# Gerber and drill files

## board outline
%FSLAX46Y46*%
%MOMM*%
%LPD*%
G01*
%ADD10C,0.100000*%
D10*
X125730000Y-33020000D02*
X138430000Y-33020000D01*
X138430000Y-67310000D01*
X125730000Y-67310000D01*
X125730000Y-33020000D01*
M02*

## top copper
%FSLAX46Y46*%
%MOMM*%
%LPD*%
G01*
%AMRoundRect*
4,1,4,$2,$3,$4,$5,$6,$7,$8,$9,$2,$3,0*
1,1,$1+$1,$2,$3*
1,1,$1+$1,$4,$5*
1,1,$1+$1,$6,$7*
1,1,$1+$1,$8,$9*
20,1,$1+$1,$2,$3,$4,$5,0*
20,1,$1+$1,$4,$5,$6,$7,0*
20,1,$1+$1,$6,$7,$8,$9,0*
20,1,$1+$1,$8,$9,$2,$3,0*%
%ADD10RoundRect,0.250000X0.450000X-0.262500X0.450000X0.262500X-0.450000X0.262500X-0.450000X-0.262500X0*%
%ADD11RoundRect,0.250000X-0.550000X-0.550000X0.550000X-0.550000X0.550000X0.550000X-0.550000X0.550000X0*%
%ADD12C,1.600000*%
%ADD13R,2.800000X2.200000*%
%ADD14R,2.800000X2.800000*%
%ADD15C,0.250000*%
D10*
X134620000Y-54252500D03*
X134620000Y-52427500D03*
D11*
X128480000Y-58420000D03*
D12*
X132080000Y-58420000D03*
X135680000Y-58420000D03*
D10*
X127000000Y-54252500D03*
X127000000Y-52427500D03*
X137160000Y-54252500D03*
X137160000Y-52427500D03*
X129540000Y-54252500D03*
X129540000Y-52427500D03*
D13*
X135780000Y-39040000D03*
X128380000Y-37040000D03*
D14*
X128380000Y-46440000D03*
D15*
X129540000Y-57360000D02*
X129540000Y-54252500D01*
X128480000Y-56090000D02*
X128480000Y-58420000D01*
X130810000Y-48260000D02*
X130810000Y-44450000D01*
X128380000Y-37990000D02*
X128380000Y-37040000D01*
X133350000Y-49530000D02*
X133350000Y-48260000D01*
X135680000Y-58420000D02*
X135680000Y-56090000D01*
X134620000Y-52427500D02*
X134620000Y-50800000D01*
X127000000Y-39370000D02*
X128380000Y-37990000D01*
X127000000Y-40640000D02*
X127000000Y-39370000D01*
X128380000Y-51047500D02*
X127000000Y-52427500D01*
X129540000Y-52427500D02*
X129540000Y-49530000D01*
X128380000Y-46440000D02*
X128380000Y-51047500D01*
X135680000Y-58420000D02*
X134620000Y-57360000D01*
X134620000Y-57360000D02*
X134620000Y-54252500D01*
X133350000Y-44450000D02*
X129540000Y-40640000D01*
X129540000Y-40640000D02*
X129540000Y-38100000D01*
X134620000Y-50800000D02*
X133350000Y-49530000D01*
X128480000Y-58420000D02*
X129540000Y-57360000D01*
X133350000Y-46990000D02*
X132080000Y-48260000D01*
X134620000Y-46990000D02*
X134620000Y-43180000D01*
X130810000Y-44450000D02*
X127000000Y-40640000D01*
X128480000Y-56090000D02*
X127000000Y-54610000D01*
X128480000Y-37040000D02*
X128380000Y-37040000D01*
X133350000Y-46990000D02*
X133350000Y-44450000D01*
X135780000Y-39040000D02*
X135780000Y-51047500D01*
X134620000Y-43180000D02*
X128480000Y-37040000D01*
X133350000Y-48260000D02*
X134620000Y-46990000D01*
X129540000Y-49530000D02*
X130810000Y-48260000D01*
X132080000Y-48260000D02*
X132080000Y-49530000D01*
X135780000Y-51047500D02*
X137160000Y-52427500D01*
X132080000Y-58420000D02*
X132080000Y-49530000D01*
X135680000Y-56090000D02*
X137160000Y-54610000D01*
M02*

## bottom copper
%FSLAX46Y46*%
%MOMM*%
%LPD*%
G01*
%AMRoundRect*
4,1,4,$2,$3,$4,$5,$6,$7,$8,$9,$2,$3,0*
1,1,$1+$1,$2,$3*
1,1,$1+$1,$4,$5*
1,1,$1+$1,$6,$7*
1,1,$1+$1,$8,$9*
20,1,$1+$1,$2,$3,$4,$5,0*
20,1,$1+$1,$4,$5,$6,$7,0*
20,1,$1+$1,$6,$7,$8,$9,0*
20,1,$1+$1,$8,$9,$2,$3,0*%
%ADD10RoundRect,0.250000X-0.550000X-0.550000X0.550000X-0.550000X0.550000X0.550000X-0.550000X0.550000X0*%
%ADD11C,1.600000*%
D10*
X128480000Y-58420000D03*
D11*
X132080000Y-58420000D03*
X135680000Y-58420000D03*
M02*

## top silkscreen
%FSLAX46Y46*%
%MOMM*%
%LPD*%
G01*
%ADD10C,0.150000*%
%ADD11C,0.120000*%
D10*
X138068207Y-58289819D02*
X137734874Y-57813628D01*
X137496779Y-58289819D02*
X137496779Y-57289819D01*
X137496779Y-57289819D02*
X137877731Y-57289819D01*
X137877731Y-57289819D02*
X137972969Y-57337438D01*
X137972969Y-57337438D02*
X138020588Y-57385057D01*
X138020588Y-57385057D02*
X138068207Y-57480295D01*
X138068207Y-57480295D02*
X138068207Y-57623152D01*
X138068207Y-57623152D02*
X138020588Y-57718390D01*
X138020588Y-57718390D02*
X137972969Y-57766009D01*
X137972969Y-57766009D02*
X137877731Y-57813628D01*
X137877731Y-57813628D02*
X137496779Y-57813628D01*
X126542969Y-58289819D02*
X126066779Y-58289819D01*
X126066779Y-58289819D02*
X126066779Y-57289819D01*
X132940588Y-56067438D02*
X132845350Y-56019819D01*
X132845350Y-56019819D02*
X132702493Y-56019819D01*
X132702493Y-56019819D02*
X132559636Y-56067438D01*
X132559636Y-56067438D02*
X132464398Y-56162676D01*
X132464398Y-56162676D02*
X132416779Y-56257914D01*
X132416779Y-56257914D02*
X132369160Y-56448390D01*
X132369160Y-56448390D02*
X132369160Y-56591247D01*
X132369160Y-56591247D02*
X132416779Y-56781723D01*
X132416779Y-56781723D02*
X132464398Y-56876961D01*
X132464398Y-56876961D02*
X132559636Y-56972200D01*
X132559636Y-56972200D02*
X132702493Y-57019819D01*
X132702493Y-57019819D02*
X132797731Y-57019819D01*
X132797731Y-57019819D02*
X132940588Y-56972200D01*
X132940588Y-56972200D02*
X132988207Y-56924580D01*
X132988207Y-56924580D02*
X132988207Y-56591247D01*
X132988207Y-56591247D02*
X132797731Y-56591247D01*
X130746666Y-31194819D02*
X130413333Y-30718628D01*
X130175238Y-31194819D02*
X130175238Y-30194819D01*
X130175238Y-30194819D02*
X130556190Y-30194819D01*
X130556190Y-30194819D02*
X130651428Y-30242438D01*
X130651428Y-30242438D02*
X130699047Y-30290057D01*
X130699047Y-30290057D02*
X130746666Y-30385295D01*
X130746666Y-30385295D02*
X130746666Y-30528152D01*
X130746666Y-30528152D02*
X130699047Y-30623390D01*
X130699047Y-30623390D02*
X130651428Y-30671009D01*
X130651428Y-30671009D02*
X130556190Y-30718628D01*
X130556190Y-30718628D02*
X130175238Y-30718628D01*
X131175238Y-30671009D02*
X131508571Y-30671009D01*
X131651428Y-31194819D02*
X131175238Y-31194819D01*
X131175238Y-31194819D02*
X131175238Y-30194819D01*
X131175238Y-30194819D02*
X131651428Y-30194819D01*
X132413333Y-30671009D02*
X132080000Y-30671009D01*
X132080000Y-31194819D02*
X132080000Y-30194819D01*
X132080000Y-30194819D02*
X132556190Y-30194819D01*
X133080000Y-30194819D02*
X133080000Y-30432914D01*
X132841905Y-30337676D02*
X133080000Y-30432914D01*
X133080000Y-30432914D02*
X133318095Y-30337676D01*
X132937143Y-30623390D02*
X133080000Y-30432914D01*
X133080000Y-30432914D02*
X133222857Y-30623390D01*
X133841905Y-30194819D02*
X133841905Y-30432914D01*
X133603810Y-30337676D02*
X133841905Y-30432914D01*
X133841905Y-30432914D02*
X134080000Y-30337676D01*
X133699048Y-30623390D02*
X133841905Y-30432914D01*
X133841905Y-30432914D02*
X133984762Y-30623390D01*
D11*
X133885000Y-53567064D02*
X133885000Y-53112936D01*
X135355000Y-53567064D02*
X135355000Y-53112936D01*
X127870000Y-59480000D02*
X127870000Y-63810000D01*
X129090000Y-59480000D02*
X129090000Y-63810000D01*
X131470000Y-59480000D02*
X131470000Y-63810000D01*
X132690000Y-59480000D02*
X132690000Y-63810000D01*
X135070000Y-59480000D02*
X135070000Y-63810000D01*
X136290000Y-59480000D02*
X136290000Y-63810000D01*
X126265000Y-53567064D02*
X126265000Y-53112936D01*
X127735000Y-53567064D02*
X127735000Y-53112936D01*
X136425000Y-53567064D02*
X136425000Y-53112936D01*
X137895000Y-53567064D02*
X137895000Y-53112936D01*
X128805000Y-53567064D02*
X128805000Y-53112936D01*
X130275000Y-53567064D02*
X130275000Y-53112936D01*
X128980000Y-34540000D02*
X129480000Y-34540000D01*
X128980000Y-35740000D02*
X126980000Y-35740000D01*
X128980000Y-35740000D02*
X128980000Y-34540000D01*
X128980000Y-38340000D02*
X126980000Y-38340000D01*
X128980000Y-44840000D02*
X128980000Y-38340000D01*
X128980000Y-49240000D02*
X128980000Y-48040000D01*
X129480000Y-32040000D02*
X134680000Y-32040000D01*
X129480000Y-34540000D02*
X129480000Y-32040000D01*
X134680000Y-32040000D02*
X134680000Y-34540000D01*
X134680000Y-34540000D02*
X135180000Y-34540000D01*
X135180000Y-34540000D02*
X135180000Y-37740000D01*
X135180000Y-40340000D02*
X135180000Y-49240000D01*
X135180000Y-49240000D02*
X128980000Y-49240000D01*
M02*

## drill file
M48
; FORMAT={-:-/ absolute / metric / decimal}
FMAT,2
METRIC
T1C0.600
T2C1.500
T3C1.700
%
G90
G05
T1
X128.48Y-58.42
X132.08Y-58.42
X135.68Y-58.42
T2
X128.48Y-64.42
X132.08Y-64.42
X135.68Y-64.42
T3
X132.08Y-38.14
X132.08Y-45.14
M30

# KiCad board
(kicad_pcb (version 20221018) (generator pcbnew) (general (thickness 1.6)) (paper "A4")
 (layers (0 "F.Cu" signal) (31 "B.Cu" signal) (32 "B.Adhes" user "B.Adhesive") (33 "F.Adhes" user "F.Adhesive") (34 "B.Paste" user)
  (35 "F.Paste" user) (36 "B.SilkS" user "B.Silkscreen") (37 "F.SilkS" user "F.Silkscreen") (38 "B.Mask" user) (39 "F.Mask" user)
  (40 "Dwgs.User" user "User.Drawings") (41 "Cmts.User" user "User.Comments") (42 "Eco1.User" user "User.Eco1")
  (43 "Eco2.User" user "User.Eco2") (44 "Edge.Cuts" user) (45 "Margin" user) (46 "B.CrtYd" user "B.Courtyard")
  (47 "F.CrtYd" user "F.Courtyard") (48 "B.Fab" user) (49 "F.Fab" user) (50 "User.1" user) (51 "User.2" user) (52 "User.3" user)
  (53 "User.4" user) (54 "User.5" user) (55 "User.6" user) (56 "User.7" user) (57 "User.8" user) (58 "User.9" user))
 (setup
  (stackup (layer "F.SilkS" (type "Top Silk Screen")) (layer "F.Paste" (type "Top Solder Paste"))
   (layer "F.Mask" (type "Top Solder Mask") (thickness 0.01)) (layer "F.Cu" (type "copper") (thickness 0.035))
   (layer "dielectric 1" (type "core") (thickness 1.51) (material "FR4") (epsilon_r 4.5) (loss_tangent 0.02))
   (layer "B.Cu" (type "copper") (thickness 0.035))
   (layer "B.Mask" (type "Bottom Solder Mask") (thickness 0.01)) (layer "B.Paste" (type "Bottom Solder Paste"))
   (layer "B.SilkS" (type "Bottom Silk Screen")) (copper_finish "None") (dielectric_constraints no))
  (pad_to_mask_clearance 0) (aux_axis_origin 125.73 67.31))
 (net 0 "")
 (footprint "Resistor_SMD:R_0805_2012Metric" (layer "F.Cu") (at 134.62 53.34 90)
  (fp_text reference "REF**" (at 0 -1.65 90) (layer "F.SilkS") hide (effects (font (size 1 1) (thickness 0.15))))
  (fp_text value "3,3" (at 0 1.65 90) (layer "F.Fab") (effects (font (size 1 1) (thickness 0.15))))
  (fp_line (start -0.227064 -0.735) (end 0.227064 -0.735) (stroke (width 0.12) (type solid)) (layer "F.SilkS"))
  (fp_line (start -0.227064 0.735) (end 0.227064 0.735) (stroke (width 0.12) (type solid)) (layer "F.SilkS"))
  (pad "1" smd roundrect (at -0.9125 0 90) (size 1.025 1.4) (layers "F.Cu" "F.Paste" "F.Mask") (roundrect_rratio 0.243902439))
  (pad "2" smd roundrect (at 0.9125 0 90) (size 1.025 1.4) (layers "F.Cu" "F.Paste" "F.Mask") (roundrect_rratio 0.243902439)))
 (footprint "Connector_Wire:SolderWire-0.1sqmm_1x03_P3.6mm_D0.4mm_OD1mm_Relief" (layer "F.Cu") (at 128.48 58.42)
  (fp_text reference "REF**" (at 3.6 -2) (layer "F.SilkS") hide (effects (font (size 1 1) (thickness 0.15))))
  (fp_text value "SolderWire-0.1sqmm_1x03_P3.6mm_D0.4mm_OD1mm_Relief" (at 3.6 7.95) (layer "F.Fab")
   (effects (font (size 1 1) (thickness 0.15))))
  (fp_line (start -0.61 1.06) (end -0.61 5.39) (stroke (width 0.12) (type solid)) (layer "F.SilkS"))
  (fp_line (start 0.61 1.06) (end 0.61 5.39) (stroke (width 0.12) (type solid)) (layer "F.SilkS"))
  (fp_line (start 2.99 1.06) (end 2.99 5.39) (stroke (width 0.12) (type solid)) (layer "F.SilkS"))
  (fp_line (start 4.21 1.06) (end 4.21 5.39) (stroke (width 0.12) (type solid)) (layer "F.SilkS"))
  (fp_line (start 6.59 1.06) (end 6.59 5.39) (stroke (width 0.12) (type solid)) (layer "F.SilkS"))
  (fp_line (start 7.81 1.06) (end 7.81 5.39) (stroke (width 0.12) (type solid)) (layer "F.SilkS"))
  (pad "" np_thru_hole circle (at 0 6) (size 1.5 1.5) (drill 1.5) (layers "*.Cu" "*.Mask"))
  (pad "" np_thru_hole circle (at 3.6 6) (size 1.5 1.5) (drill 1.5) (layers "*.Cu" "*.Mask"))
  (pad "" np_thru_hole circle (at 7.2 6) (size 1.5 1.5) (drill 1.5) (layers "*.Cu" "*.Mask"))
  (pad "1" thru_hole roundrect (at 0 0) (size 1.6 1.6) (drill 0.6) (layers "*.Cu" "*.Mask") (roundrect_rratio 0.15625))
  (pad "2" thru_hole circle (at 3.6 0) (size 1.6 1.6) (drill 0.6) (layers "*.Cu" "*.Mask"))
  (pad "3" thru_hole circle (at 7.2 0) (size 1.6 1.6) (drill 0.6) (layers "*.Cu" "*.Mask")))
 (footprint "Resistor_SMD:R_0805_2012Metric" (layer "F.Cu") (at 127 53.34 90)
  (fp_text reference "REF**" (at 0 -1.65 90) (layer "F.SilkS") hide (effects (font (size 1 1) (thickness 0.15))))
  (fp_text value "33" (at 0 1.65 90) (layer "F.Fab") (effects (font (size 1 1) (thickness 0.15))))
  (fp_line (start -0.227064 -0.735) (end 0.227064 -0.735) (stroke (width 0.12) (type solid)) (layer "F.SilkS"))
  (fp_line (start -0.227064 0.735) (end 0.227064 0.735) (stroke (width 0.12) (type solid)) (layer "F.SilkS"))
  (pad "1" smd roundrect (at -0.9125 0 90) (size 1.025 1.4) (layers "F.Cu" "F.Paste" "F.Mask") (roundrect_rratio 0.243902439))
  (pad "2" smd roundrect (at 0.9125 0 90) (size 1.025 1.4) (layers "F.Cu" "F.Paste" "F.Mask") (roundrect_rratio 0.243902439)))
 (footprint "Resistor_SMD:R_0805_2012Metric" (layer "F.Cu") (at 137.16 53.34 90)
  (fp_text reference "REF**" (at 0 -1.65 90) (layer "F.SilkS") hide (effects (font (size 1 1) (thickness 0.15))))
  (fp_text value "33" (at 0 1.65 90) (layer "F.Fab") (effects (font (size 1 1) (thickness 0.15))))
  (fp_line (start -0.227064 -0.735) (end 0.227064 -0.735) (stroke (width 0.12) (type solid)) (layer "F.SilkS"))
  (fp_line (start -0.227064 0.735) (end 0.227064 0.735) (stroke (width 0.12) (type solid)) (layer "F.SilkS"))
  (pad "1" smd roundrect (at -0.9125 0 90) (size 1.025 1.4) (layers "F.Cu" "F.Paste" "F.Mask") (roundrect_rratio 0.243902439))
  (pad "2" smd roundrect (at 0.9125 0 90) (size 1.025 1.4) (layers "F.Cu" "F.Paste" "F.Mask") (roundrect_rratio 0.243902439)))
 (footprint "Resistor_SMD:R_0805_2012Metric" (layer "F.Cu") (at 129.54 53.34 90)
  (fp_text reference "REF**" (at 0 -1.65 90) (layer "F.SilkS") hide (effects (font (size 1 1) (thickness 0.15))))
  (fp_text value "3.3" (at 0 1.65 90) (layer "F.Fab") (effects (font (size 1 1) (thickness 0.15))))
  (fp_line (start -0.227064 -0.735) (end 0.227064 -0.735) (stroke (width 0.12) (type solid)) (layer "F.SilkS"))
  (fp_line (start -0.227064 0.735) (end 0.227064 0.735) (stroke (width 0.12) (type solid)) (layer "F.SilkS"))
  (pad "1" smd roundrect (at -0.9125 0 90) (size 1.025 1.4) (layers "F.Cu" "F.Paste" "F.Mask") (roundrect_rratio 0.243902439))
  (pad "2" smd roundrect (at 0.9125 0 90) (size 1.025 1.4) (layers "F.Cu" "F.Paste" "F.Mask") (roundrect_rratio 0.243902439)))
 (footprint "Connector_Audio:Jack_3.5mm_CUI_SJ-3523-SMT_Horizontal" (layer "F.Cu") (at 132.08 40.64)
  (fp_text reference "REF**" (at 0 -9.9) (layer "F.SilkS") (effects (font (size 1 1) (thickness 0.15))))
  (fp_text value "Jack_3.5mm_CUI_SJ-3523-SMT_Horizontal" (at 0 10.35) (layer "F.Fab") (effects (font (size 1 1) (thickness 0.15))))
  (fp_line (start -3.1 -6.1) (end -2.6 -6.1) (stroke (width 0.12) (type solid)) (layer "F.SilkS"))
  (fp_line (start -3.1 -4.9) (end -5.1 -4.9) (stroke (width 0.12) (type solid)) (layer "F.SilkS"))
  (fp_line (start -3.1 -4.9) (end -3.1 -6.1) (stroke (width 0.12) (type solid)) (layer "F.SilkS"))
  (fp_line (start -3.1 -2.3) (end -5.1 -2.3) (stroke (width 0.12) (type solid)) (layer "F.SilkS"))
  (fp_line (start -3.1 4.2) (end -3.1 -2.3) (stroke (width 0.12) (type solid)) (layer "F.SilkS"))
  (fp_line (start -3.1 8.6) (end -3.1 7.4) (stroke (width 0.12) (type solid)) (layer "F.SilkS"))
  (fp_line (start -2.6 -8.6) (end 2.6 -8.6) (stroke (width 0.12) (type solid)) (layer "F.SilkS"))
  (fp_line (start -2.6 -6.1) (end -2.6 -8.6) (stroke (width 0.12) (type solid)) (layer "F.SilkS"))
  (fp_line (start 2.6 -8.6) (end 2.6 -6.1) (stroke (width 0.12) (type solid)) (layer "F.SilkS"))
  (fp_line (start 2.6 -6.1) (end 3.1 -6.1) (stroke (width 0.12) (type solid)) (layer "F.SilkS"))
  (fp_line (start 3.1 -6.1) (end 3.1 -2.9) (stroke (width 0.12) (type solid)) (layer "F.SilkS"))
  (fp_line (start 3.1 -0.3) (end 3.1 8.6) (stroke (width 0.12) (type solid)) (layer "F.SilkS"))
  (fp_line (start 3.1 8.6) (end -3.1 8.6) (stroke (width 0.12) (type solid)) (layer "F.SilkS"))
  (pad "" np_thru_hole circle (at 0 -2.5) (size 1.7 1.7) (drill 1.7) (layers "*.Cu" "*.Mask"))
  (pad "" np_thru_hole circle (at 0 4.5) (size 1.7 1.7) (drill 1.7) (layers "*.Cu" "*.Mask"))
  (pad "R" smd rect (at 3.7 -1.6) (size 2.8 2.2) (layers "F.Cu" "F.Paste" "F.Mask"))
  (pad "S" smd rect (at -3.7 -3.6) (size 2.8 2.2) (layers "F.Cu" "F.Paste" "F.Mask"))
  (pad "T" smd rect (at -3.7 5.8) (size 2.8 2.8) (layers "F.Cu" "F.Paste" "F.Mask")))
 (gr_poly
  (pts (xy 125.73 33.02) (xy 138.43 33.02) (xy 138.43 67.31) (xy 125.73 67.31)) (stroke (width 0.1) (type solid)) (fill none)
  (layer "Edge.Cuts"))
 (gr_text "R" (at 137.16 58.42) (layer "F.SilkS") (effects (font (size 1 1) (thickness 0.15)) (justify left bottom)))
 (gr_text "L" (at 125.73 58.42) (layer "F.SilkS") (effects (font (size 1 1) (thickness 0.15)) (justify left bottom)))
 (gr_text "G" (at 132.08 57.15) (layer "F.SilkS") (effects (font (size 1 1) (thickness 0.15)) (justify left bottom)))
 (segment (start 129.54 57.36) (end 129.54 54.2525) (width 0.25) (layer "F.Cu") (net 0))
 (segment (start 128.48 56.09) (end 128.48 58.42) (width 0.25) (layer "F.Cu") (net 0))
 (segment (start 130.81 48.26) (end 130.81 44.45) (width 0.25) (layer "F.Cu") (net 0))
 (segment (start 128.38 37.99) (end 128.38 37.04) (width 0.25) (layer "F.Cu") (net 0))
 (segment (start 133.35 49.53) (end 133.35 48.26) (width 0.25) (layer "F.Cu") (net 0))
 (segment (start 135.68 58.42) (end 135.68 56.09) (width 0.25) (layer "F.Cu") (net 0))
 (segment (start 134.62 52.4275) (end 134.62 50.8) (width 0.25) (layer "F.Cu") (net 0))
 (segment (start 127 39.37) (end 128.38 37.99) (width 0.25) (layer "F.Cu") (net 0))
 (segment (start 127 40.64) (end 127 39.37) (width 0.25) (layer "F.Cu") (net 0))
 (segment (start 128.38 51.0475) (end 127 52.4275) (width 0.25) (layer "F.Cu") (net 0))
 (segment (start 129.54 52.4275) (end 129.54 49.53) (width 0.25) (layer "F.Cu") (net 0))
 (segment (start 128.38 46.44) (end 128.38 51.0475) (width 0.25) (layer "F.Cu") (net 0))
 (segment (start 135.68 58.42) (end 134.62 57.36) (width 0.25) (layer "F.Cu") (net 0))
 (segment (start 134.62 57.36) (end 134.62 54.2525) (width 0.25) (layer "F.Cu") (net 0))
 (segment (start 133.35 44.45) (end 129.54 40.64) (width 0.25) (layer "F.Cu") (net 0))
 (segment (start 129.54 40.64) (end 129.54 38.1) (width 0.25) (layer "F.Cu") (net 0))
 (segment (start 134.62 50.8) (end 133.35 49.53) (width 0.25) (layer "F.Cu") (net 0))
 (segment (start 128.48 58.42) (end 129.54 57.36) (width 0.25) (layer "F.Cu") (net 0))
 (segment (start 133.35 46.99) (end 132.08 48.26) (width 0.25) (layer "F.Cu") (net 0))
 (segment (start 134.62 46.99) (end 134.62 43.18) (width 0.25) (layer "F.Cu") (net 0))
 (segment (start 130.81 44.45) (end 127 40.64) (width 0.25) (layer "F.Cu") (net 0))
 (segment (start 128.48 56.09) (end 127 54.61) (width 0.25) (layer "F.Cu") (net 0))
 (segment (start 128.48 37.04) (end 128.38 37.04) (width 0.25) (layer "F.Cu") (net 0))
 (segment (start 133.35 46.99) (end 133.35 44.45) (width 0.25) (layer "F.Cu") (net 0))
 (segment (start 135.78 39.04) (end 135.78 51.0475) (width 0.25) (layer "F.Cu") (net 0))
 (segment (start 134.62 43.18) (end 128.48 37.04) (width 0.25) (layer "F.Cu") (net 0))
 (segment (start 133.35 48.26) (end 134.62 46.99) (width 0.25) (layer "F.Cu") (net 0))
 (segment (start 129.54 49.53) (end 130.81 48.26) (width 0.25) (layer "F.Cu") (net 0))
 (segment (start 132.08 48.26) (end 132.08 49.53) (width 0.25) (layer "F.Cu") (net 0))
 (segment (start 135.78 51.0475) (end 137.16 52.4275) (width 0.25) (layer "F.Cu") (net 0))
 (segment (start 132.08 58.42) (end 132.08 49.53) (width 0.25) (layer "F.Cu") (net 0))
 (segment (start 135.68 56.09) (end 137.16 54.61) (width 0.25) (layer "F.Cu") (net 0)))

